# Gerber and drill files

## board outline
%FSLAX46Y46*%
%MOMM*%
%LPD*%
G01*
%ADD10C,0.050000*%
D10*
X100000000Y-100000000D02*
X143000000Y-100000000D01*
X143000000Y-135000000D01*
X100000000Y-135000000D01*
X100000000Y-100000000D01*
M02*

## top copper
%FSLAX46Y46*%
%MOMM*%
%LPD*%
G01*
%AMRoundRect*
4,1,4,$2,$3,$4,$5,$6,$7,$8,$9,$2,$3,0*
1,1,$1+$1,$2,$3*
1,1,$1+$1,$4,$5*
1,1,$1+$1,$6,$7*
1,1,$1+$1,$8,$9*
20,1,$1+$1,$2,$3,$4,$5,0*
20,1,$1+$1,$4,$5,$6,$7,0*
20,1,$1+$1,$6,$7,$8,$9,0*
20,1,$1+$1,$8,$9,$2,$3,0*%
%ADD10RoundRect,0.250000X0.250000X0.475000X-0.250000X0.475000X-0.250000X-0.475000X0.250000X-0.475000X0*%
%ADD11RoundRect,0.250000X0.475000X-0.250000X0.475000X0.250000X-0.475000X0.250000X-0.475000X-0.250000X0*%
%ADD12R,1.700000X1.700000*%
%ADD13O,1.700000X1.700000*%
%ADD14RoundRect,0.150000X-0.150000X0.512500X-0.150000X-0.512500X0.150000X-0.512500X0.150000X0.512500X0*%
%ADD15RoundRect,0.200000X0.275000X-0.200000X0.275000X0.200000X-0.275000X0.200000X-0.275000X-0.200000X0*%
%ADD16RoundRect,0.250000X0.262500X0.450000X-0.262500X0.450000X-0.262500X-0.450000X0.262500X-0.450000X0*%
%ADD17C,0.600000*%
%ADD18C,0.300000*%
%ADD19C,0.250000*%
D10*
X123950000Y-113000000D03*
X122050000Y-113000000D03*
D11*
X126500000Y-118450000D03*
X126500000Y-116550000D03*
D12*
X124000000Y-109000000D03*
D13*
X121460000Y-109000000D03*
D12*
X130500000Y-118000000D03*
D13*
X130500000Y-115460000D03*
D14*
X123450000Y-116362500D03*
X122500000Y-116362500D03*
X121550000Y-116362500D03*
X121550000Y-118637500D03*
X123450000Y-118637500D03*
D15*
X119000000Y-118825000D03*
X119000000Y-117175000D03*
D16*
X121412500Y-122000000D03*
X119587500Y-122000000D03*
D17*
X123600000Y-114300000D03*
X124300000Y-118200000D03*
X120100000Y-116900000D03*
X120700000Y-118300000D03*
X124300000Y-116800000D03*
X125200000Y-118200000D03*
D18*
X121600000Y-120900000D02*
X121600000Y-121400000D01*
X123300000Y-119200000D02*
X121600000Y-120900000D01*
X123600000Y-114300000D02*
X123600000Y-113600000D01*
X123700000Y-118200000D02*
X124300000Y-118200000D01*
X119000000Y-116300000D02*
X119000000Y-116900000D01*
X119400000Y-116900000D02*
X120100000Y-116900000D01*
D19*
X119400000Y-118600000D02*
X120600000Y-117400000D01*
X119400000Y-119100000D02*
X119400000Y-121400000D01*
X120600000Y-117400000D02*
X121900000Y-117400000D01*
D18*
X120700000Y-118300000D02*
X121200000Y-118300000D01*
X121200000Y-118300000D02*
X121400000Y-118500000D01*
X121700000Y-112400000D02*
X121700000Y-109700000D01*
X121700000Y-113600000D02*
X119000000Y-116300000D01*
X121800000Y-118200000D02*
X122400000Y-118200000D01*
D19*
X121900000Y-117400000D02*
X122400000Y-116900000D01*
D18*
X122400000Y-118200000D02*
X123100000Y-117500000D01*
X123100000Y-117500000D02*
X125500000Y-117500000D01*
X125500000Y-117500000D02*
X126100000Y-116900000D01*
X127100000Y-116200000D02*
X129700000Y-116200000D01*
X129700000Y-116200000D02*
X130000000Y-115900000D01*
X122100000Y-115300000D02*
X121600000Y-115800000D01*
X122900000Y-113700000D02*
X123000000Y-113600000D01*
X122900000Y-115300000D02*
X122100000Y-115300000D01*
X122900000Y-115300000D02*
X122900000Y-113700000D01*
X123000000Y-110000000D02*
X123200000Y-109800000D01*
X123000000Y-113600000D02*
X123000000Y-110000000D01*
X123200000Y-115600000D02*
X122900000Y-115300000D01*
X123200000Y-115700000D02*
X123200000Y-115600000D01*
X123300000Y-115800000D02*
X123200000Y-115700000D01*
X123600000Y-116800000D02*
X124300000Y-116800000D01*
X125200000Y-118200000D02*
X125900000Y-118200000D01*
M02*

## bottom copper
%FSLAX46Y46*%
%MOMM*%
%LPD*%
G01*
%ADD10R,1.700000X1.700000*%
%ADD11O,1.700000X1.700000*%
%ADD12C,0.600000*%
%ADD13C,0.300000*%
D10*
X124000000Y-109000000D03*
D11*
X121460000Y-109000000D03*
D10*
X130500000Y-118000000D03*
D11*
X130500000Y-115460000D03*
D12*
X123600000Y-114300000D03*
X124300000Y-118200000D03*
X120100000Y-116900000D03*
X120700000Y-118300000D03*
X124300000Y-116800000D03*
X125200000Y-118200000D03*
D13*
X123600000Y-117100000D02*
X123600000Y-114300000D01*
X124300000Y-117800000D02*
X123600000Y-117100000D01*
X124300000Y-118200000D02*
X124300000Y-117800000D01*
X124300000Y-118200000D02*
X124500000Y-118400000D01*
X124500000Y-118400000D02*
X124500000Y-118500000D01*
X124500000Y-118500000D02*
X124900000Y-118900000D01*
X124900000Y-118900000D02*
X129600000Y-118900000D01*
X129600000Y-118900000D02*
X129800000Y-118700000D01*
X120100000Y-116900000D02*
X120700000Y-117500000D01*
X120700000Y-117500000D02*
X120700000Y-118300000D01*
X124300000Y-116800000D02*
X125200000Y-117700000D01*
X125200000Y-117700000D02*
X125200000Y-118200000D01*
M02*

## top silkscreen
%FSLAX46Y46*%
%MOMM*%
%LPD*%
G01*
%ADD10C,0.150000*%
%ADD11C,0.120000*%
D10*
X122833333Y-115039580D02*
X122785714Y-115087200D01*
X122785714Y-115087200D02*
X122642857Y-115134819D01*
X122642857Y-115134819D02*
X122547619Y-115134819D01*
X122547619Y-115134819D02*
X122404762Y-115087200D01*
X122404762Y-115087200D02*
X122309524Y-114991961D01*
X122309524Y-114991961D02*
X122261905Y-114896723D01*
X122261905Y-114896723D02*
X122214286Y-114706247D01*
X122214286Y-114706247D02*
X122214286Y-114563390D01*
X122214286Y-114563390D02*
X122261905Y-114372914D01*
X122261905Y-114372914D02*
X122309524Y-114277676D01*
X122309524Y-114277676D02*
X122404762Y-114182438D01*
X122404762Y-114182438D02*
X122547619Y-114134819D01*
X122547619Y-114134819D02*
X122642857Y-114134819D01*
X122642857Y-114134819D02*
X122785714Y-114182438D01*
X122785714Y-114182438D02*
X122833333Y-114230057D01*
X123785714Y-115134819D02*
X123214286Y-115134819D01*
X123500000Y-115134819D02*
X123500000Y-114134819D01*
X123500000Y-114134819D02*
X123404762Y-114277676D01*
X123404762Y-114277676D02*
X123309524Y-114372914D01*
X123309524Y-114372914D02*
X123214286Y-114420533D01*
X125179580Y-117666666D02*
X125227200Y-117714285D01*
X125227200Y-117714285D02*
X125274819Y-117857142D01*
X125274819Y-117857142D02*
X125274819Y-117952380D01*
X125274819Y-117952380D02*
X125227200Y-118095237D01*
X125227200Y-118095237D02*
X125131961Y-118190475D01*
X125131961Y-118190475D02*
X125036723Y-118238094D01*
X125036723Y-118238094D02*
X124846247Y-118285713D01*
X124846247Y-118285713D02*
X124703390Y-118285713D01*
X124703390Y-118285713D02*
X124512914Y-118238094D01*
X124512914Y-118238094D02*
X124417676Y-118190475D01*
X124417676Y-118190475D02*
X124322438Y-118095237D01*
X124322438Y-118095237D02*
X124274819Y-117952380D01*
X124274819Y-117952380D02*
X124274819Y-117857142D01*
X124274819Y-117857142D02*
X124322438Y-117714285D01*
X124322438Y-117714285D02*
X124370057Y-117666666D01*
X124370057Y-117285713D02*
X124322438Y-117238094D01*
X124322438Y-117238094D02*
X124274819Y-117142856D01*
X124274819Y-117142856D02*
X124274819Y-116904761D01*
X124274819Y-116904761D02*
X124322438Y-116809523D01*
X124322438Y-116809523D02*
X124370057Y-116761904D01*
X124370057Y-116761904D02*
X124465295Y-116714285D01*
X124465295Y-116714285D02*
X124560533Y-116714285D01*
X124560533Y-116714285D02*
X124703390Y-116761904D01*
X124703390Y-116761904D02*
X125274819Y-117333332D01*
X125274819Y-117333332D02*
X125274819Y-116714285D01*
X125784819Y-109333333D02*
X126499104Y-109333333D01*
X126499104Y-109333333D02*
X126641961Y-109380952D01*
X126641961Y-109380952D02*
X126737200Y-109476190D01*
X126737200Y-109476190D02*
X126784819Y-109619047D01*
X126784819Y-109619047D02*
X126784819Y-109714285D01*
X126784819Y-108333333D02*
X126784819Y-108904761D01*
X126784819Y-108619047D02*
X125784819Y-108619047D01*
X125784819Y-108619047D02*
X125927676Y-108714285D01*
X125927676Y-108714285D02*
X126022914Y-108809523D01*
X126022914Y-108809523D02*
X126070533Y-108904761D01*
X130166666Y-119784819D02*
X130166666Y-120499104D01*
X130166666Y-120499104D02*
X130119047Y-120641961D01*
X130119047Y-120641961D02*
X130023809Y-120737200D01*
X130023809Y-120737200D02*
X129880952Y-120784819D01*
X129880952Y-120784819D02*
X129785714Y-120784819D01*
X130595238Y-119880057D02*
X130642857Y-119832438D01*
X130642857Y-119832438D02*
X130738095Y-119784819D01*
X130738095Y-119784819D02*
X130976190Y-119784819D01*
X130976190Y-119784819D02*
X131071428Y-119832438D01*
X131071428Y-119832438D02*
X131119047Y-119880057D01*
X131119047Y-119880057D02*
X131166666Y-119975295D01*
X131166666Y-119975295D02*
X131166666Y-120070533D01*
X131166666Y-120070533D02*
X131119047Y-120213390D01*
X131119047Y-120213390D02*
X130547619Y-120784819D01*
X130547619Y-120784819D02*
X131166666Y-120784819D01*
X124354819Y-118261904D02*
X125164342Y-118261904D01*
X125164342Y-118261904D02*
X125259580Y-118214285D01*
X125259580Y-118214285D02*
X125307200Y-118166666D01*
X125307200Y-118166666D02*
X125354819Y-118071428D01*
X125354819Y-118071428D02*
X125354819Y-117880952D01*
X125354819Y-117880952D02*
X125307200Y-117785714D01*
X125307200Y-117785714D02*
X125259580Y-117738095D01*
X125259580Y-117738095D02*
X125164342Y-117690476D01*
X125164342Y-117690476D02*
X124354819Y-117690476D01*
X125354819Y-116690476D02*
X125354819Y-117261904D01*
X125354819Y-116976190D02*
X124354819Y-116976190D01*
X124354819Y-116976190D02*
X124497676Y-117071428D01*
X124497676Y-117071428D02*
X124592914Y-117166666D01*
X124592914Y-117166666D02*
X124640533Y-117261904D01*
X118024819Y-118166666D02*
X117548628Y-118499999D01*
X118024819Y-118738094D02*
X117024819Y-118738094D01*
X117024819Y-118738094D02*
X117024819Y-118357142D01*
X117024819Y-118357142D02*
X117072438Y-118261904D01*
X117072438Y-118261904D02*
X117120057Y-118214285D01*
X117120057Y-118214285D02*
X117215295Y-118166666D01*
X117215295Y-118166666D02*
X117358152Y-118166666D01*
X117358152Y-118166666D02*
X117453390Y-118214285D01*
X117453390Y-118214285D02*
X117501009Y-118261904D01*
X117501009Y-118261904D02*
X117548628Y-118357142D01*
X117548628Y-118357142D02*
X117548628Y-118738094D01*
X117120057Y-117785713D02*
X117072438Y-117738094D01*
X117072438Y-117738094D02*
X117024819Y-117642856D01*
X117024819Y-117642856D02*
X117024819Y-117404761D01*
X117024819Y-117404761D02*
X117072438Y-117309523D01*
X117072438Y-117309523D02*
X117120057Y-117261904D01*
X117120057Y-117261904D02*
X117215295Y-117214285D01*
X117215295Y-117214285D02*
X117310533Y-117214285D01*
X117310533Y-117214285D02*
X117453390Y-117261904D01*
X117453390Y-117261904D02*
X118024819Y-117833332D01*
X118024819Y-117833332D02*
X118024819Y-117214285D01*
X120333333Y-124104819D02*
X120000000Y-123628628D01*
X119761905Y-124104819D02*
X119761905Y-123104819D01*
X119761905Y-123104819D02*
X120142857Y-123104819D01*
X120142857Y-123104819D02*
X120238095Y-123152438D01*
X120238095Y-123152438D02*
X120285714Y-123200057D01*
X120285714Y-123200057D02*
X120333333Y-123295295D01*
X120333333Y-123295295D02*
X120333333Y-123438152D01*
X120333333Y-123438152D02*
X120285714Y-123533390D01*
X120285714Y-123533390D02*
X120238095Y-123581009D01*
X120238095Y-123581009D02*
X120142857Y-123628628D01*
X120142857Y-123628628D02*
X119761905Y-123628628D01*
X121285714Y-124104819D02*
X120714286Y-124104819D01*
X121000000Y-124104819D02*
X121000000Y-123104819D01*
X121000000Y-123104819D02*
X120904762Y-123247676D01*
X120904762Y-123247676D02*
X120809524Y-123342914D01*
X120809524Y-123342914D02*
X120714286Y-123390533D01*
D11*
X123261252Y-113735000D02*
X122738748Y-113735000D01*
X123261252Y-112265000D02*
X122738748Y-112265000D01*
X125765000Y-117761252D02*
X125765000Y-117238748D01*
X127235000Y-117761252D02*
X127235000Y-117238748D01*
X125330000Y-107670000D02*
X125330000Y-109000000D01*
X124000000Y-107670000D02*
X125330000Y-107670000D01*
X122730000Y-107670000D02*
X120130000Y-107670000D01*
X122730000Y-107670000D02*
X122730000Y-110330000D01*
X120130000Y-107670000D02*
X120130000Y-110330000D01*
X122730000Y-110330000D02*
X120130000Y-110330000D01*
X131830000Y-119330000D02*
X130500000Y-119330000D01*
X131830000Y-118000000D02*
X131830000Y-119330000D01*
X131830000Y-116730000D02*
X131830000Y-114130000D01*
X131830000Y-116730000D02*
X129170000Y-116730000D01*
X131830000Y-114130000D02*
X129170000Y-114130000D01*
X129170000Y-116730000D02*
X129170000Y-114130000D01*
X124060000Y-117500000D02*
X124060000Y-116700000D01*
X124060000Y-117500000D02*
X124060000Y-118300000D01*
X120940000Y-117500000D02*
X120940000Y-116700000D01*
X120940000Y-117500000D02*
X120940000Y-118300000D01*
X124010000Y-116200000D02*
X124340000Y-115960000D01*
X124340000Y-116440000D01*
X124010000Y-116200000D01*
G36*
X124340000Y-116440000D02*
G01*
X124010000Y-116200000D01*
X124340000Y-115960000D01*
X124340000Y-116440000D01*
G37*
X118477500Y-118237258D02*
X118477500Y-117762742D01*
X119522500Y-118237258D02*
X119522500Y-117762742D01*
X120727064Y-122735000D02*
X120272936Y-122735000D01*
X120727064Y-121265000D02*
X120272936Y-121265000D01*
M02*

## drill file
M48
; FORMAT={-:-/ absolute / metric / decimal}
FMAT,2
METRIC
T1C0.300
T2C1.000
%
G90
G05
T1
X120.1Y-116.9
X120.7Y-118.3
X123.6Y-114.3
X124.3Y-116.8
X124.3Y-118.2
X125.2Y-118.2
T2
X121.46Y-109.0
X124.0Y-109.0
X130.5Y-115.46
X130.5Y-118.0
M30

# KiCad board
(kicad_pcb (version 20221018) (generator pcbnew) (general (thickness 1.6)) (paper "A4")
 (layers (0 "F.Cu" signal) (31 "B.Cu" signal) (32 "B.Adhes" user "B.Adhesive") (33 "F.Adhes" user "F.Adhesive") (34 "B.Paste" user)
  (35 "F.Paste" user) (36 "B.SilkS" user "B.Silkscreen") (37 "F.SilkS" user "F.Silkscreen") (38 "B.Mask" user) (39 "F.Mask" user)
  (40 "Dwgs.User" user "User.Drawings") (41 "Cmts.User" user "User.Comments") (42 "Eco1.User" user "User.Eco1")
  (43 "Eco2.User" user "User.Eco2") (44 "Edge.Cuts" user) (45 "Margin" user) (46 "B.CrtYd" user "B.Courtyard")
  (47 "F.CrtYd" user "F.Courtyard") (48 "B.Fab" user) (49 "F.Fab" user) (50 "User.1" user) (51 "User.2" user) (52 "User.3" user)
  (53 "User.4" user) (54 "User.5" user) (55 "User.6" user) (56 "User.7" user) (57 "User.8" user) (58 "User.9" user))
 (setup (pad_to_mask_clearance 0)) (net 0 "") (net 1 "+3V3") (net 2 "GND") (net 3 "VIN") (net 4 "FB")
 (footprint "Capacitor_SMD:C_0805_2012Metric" (layer "F.Cu") (at 123 113 180)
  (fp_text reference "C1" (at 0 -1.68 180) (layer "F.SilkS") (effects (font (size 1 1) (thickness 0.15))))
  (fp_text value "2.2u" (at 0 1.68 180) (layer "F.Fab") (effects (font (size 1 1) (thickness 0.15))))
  (fp_line (start -0.261252 -0.735) (end 0.261252 -0.735) (stroke (width 0.12) (type solid)) (layer "F.SilkS"))
  (fp_line (start -0.261252 0.735) (end 0.261252 0.735) (stroke (width 0.12) (type solid)) (layer "F.SilkS"))
  (pad "1" smd roundrect (at -0.95 0 180) (size 1 1.45) (layers "F.Cu" "F.Paste" "F.Mask") (roundrect_rratio 0.25) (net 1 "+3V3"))
  (pad "2" smd roundrect (at 0.95 0 180) (size 1 1.45) (layers "F.Cu" "F.Paste" "F.Mask") (roundrect_rratio 0.25) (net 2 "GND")))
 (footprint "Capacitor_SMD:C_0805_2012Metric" (layer "F.Cu") (at 126.5 117.5 90)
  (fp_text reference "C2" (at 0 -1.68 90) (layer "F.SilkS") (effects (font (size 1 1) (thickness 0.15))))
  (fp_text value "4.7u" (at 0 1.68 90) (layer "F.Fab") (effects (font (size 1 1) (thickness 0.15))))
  (fp_line (start -0.261252 -0.735) (end 0.261252 -0.735) (stroke (width 0.12) (type solid)) (layer "F.SilkS"))
  (fp_line (start -0.261252 0.735) (end 0.261252 0.735) (stroke (width 0.12) (type solid)) (layer "F.SilkS"))
  (pad "1" smd roundrect (at -0.95 0 90) (size 1 1.45) (layers "F.Cu" "F.Paste" "F.Mask") (roundrect_rratio 0.25) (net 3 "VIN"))
  (pad "2" smd roundrect (at 0.95 0 90) (size 1 1.45) (layers "F.Cu" "F.Paste" "F.Mask") (roundrect_rratio 0.25) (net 2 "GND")))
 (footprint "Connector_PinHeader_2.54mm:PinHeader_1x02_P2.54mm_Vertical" (layer "F.Cu") (at 124 109 -90)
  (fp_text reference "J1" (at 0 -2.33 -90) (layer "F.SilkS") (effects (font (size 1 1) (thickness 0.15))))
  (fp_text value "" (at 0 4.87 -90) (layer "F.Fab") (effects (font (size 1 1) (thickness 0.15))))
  (fp_line (start -1.33 -1.33) (end 0 -1.33) (stroke (width 0.12) (type solid)) (layer "F.SilkS"))
  (fp_line (start -1.33 0) (end -1.33 -1.33) (stroke (width 0.12) (type solid)) (layer "F.SilkS"))
  (fp_line (start -1.33 1.27) (end -1.33 3.87) (stroke (width 0.12) (type solid)) (layer "F.SilkS"))
  (fp_line (start -1.33 1.27) (end 1.33 1.27) (stroke (width 0.12) (type solid)) (layer "F.SilkS"))
  (fp_line (start -1.33 3.87) (end 1.33 3.87) (stroke (width 0.12) (type solid)) (layer "F.SilkS"))
  (fp_line (start 1.33 1.27) (end 1.33 3.87) (stroke (width 0.12) (type solid)) (layer "F.SilkS"))
  (pad "1" thru_hole rect (at 0 0 270) (size 1.7 1.7) (drill 1) (layers "*.Cu" "*.Mask") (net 3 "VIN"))
  (pad "2" thru_hole oval (at 0 2.54 270) (size 1.7 1.7) (drill 1) (layers "*.Cu" "*.Mask") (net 2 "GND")))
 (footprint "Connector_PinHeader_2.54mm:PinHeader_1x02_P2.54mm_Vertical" (layer "F.Cu") (at 130.5 118 180)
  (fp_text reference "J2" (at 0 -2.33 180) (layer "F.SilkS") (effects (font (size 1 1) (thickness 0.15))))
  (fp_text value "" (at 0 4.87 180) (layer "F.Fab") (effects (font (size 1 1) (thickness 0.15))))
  (fp_line (start -1.33 -1.33) (end 0 -1.33) (stroke (width 0.12) (type solid)) (layer "F.SilkS"))
  (fp_line (start -1.33 0) (end -1.33 -1.33) (stroke (width 0.12) (type solid)) (layer "F.SilkS"))
  (fp_line (start -1.33 1.27) (end -1.33 3.87) (stroke (width 0.12) (type solid)) (layer "F.SilkS"))
  (fp_line (start -1.33 1.27) (end 1.33 1.27) (stroke (width 0.12) (type solid)) (layer "F.SilkS"))
  (fp_line (start -1.33 3.87) (end 1.33 3.87) (stroke (width 0.12) (type solid)) (layer "F.SilkS"))
  (fp_line (start 1.33 1.27) (end 1.33 3.87) (stroke (width 0.12) (type solid)) (layer "F.SilkS"))
  (pad "1" thru_hole rect (at 0 0 180) (size 1.7 1.7) (drill 1) (layers "*.Cu" "*.Mask") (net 1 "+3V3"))
  (pad "2" thru_hole oval (at 0 2.54 180) (size 1.7 1.7) (drill 1) (layers "*.Cu" "*.Mask") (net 2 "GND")))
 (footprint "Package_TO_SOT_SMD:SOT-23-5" (layer "F.Cu") (at 122.5 117.5 -90)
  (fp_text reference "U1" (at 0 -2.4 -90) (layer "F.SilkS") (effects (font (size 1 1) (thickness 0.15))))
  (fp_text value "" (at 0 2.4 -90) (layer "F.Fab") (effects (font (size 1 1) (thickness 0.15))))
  (fp_line (start 0 -1.56) (end -0.8 -1.56) (stroke (width 0.12) (type solid)) (layer "F.SilkS"))
  (fp_line (start 0 -1.56) (end 0.8 -1.56) (stroke (width 0.12) (type solid)) (layer "F.SilkS"))
  (fp_line (start 0 1.56) (end -0.8 1.56) (stroke (width 0.12) (type solid)) (layer "F.SilkS"))
  (fp_line (start 0 1.56) (end 0.8 1.56) (stroke (width 0.12) (type solid)) (layer "F.SilkS"))
  (fp_poly
   (pts (xy -1.3 -1.51) (xy -1.54 -1.84) (xy -1.06 -1.84) (xy -1.3 -1.51)) (stroke (width 0.12) (type solid)) (fill solid) (layer "F.SilkS"))
  (pad "1" smd roundrect (at -1.1375 -0.95 270) (size 1.325 0.6) (layers "F.Cu" "F.Paste" "F.Mask") (roundrect_rratio 0.25) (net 3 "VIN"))
  (pad "2" smd roundrect (at -1.1375 0 270) (size 1.325 0.6) (layers "F.Cu" "F.Paste" "F.Mask") (roundrect_rratio 0.25) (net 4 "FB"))
  (pad "3" smd roundrect (at -1.1375 0.95 270) (size 1.325 0.6) (layers "F.Cu" "F.Paste" "F.Mask") (roundrect_rratio 0.25) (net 3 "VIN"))
  (pad "4" smd roundrect (at 1.1375 0.95 270) (size 1.325 0.6) (layers "F.Cu" "F.Paste" "F.Mask") (roundrect_rratio 0.25) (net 2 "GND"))
  (pad "5" smd roundrect (at 1.1375 -0.95 270) (size 1.325 0.6) (layers "F.Cu" "F.Paste" "F.Mask") (roundrect_rratio 0.25) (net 1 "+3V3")))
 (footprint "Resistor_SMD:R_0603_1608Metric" (layer "F.Cu") (at 119 118 90)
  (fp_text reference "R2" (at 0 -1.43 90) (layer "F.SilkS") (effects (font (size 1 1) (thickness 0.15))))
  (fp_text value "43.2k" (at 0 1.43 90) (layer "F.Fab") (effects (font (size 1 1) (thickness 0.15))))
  (fp_line (start -0.237258 -0.5225) (end 0.237258 -0.5225) (stroke (width 0.12) (type solid)) (layer "F.SilkS"))
  (fp_line (start -0.237258 0.5225) (end 0.237258 0.5225) (stroke (width 0.12) (type solid)) (layer "F.SilkS"))
  (pad "1" smd roundrect (at -0.825 0 90) (size 0.8 0.95) (layers "F.Cu" "F.Paste" "F.Mask") (roundrect_rratio 0.25) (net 4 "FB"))
  (pad "2" smd roundrect (at 0.825 0 90) (size 0.8 0.95) (layers "F.Cu" "F.Paste" "F.Mask") (roundrect_rratio 0.25) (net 2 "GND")))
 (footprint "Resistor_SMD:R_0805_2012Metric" (layer "F.Cu") (at 120.5 122 180)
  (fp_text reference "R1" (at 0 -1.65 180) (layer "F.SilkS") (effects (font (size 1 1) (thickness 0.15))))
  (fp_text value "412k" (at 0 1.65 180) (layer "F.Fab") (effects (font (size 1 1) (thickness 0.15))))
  (fp_line (start -0.227064 -0.735) (end 0.227064 -0.735) (stroke (width 0.12) (type solid)) (layer "F.SilkS"))
  (fp_line (start -0.227064 0.735) (end 0.227064 0.735) (stroke (width 0.12) (type solid)) (layer "F.SilkS"))
  (pad "1" smd roundrect (at -0.9125 0 180) (size 1.025 1.4) (layers "F.Cu" "F.Paste" "F.Mask") (roundrect_rratio 0.243902) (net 1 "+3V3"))
  (pad "2" smd roundrect (at 0.9125 0 180) (size 1.025 1.4) (layers "F.Cu" "F.Paste" "F.Mask") (roundrect_rratio 0.243902) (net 4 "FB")))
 (gr_rect (start 100 100) (end 143 135) (stroke (width 0.05) (type default)) (fill none) (layer "Edge.Cuts"))
 (segment (start 121.6 120.9) (end 121.6 121.4) (width 0.3) (layer "F.Cu") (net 1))
 (segment (start 123.3 119.2) (end 121.6 120.9) (width 0.3) (layer "F.Cu") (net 1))
 (segment (start 123.6 114.3) (end 123.6 113.6) (width 0.3) (layer "F.Cu") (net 1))
 (segment (start 123.7 118.2) (end 124.3 118.2) (width 0.3) (layer "F.Cu") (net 1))
 (via (at 123.6 114.3) (size 0.6) (drill 0.3) (layers "F.Cu" "B.Cu") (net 1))
 (via (at 124.3 118.2) (size 0.6) (drill 0.3) (layers "F.Cu" "B.Cu") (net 1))
 (segment (start 119 116.3) (end 119 116.9) (width 0.3) (layer "F.Cu") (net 2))
 (segment (start 119.4 116.9) (end 120.1 116.9) (width 0.3) (layer "F.Cu") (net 2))
 (segment (start 119.4 118.6) (end 120.6 117.4) (width 0.25) (layer "F.Cu") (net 4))
 (segment (start 119.4 119.1) (end 119.4 121.4) (width 0.25) (layer "F.Cu") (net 4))
 (segment (start 120.6 117.4) (end 121.9 117.4) (width 0.25) (layer "F.Cu") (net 4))
 (segment (start 120.7 118.3) (end 121.2 118.3) (width 0.3) (layer "F.Cu") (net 2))
 (segment (start 121.2 118.3) (end 121.4 118.5) (width 0.3) (layer "F.Cu") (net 2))
 (segment (start 121.7 112.4) (end 121.7 109.7) (width 0.3) (layer "F.Cu") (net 2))
 (segment (start 121.7 113.6) (end 119 116.3) (width 0.3) (layer "F.Cu") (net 2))
 (segment (start 121.8 118.2) (end 122.4 118.2) (width 0.3) (layer "F.Cu") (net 2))
 (segment (start 121.9 117.4) (end 122.4 116.9) (width 0.25) (layer "F.Cu") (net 4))
 (segment (start 122.4 118.2) (end 123.1 117.5) (width 0.3) (layer "F.Cu") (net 2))
 (segment (start 123.1 117.5) (end 125.5 117.5) (width 0.3) (layer "F.Cu") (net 2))
 (segment (start 123.6 117.1) (end 123.6 114.3) (width 0.3) (layer "B.Cu") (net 1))
 (segment (start 124.3 117.8) (end 123.6 117.1) (width 0.3) (layer "B.Cu") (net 1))
 (segment (start 124.3 118.2) (end 124.3 117.8) (width 0.3) (layer "B.Cu") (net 1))
 (segment (start 124.3 118.2) (end 124.5 118.4) (width 0.3) (layer "B.Cu") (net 1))
 (segment (start 124.5 118.4) (end 124.5 118.5) (width 0.3) (layer "B.Cu") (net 1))
 (segment (start 124.5 118.5) (end 124.9 118.9) (width 0.3) (layer "B.Cu") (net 1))
 (segment (start 124.9 118.9) (end 129.6 118.9) (width 0.3) (layer "B.Cu") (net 1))
 (segment (start 125.5 117.5) (end 126.1 116.9) (width 0.3) (layer "F.Cu") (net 2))
 (segment (start 127.1 116.2) (end 129.7 116.2) (width 0.3) (layer "F.Cu") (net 2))
 (segment (start 129.6 118.9) (end 129.8 118.7) (width 0.3) (layer "B.Cu") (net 1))
 (segment (start 129.7 116.2) (end 130 115.9) (width 0.3) (layer "F.Cu") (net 2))
 (via (at 120.1 116.9) (size 0.6) (drill 0.3) (layers "F.Cu" "B.Cu") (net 2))
 (via (at 120.7 118.3) (size 0.6) (drill 0.3) (layers "F.Cu" "B.Cu") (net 2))
 (segment (start 120.1 116.9) (end 120.7 117.5) (width 0.3) (layer "B.Cu") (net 2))
 (segment (start 120.7 117.5) (end 120.7 118.3) (width 0.3) (layer "B.Cu") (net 2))
 (segment (start 122.1 115.3) (end 121.6 115.8) (width 0.3) (layer "F.Cu") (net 3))
 (segment (start 122.9 113.7) (end 123 113.6) (width 0.3) (layer "F.Cu") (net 3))
 (segment (start 122.9 115.3) (end 122.1 115.3) (width 0.3) (layer "F.Cu") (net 3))
 (segment (start 122.9 115.3) (end 122.9 113.7) (width 0.3) (layer "F.Cu") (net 3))
 (segment (start 123 110) (end 123.2 109.8) (width 0.3) (layer "F.Cu") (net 3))
 (segment (start 123 113.6) (end 123 110) (width 0.3) (layer "F.Cu") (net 3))
 (segment (start 123.2 115.6) (end 122.9 115.3) (width 0.3) (layer "F.Cu") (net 3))
 (segment (start 123.2 115.7) (end 123.2 115.6) (width 0.3) (layer "F.Cu") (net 3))
 (segment (start 123.3 115.8) (end 123.2 115.7) (width 0.3) (layer "F.Cu") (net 3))
 (segment (start 123.6 116.8) (end 124.3 116.8) (width 0.3) (layer "F.Cu") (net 3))
 (segment (start 125.2 118.2) (end 125.9 118.2) (width 0.3) (layer "F.Cu") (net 3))
 (via (at 124.3 116.8) (size 0.6) (drill 0.3) (layers "F.Cu" "B.Cu") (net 3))
 (via (at 125.2 118.2) (size 0.6) (drill 0.3) (layers "F.Cu" "B.Cu") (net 3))
 (segment (start 124.3 116.8) (end 125.2 117.7) (width 0.3) (layer "B.Cu") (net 3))
 (segment (start 125.2 117.7) (end 125.2 118.2) (width 0.3) (layer "B.Cu") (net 3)))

